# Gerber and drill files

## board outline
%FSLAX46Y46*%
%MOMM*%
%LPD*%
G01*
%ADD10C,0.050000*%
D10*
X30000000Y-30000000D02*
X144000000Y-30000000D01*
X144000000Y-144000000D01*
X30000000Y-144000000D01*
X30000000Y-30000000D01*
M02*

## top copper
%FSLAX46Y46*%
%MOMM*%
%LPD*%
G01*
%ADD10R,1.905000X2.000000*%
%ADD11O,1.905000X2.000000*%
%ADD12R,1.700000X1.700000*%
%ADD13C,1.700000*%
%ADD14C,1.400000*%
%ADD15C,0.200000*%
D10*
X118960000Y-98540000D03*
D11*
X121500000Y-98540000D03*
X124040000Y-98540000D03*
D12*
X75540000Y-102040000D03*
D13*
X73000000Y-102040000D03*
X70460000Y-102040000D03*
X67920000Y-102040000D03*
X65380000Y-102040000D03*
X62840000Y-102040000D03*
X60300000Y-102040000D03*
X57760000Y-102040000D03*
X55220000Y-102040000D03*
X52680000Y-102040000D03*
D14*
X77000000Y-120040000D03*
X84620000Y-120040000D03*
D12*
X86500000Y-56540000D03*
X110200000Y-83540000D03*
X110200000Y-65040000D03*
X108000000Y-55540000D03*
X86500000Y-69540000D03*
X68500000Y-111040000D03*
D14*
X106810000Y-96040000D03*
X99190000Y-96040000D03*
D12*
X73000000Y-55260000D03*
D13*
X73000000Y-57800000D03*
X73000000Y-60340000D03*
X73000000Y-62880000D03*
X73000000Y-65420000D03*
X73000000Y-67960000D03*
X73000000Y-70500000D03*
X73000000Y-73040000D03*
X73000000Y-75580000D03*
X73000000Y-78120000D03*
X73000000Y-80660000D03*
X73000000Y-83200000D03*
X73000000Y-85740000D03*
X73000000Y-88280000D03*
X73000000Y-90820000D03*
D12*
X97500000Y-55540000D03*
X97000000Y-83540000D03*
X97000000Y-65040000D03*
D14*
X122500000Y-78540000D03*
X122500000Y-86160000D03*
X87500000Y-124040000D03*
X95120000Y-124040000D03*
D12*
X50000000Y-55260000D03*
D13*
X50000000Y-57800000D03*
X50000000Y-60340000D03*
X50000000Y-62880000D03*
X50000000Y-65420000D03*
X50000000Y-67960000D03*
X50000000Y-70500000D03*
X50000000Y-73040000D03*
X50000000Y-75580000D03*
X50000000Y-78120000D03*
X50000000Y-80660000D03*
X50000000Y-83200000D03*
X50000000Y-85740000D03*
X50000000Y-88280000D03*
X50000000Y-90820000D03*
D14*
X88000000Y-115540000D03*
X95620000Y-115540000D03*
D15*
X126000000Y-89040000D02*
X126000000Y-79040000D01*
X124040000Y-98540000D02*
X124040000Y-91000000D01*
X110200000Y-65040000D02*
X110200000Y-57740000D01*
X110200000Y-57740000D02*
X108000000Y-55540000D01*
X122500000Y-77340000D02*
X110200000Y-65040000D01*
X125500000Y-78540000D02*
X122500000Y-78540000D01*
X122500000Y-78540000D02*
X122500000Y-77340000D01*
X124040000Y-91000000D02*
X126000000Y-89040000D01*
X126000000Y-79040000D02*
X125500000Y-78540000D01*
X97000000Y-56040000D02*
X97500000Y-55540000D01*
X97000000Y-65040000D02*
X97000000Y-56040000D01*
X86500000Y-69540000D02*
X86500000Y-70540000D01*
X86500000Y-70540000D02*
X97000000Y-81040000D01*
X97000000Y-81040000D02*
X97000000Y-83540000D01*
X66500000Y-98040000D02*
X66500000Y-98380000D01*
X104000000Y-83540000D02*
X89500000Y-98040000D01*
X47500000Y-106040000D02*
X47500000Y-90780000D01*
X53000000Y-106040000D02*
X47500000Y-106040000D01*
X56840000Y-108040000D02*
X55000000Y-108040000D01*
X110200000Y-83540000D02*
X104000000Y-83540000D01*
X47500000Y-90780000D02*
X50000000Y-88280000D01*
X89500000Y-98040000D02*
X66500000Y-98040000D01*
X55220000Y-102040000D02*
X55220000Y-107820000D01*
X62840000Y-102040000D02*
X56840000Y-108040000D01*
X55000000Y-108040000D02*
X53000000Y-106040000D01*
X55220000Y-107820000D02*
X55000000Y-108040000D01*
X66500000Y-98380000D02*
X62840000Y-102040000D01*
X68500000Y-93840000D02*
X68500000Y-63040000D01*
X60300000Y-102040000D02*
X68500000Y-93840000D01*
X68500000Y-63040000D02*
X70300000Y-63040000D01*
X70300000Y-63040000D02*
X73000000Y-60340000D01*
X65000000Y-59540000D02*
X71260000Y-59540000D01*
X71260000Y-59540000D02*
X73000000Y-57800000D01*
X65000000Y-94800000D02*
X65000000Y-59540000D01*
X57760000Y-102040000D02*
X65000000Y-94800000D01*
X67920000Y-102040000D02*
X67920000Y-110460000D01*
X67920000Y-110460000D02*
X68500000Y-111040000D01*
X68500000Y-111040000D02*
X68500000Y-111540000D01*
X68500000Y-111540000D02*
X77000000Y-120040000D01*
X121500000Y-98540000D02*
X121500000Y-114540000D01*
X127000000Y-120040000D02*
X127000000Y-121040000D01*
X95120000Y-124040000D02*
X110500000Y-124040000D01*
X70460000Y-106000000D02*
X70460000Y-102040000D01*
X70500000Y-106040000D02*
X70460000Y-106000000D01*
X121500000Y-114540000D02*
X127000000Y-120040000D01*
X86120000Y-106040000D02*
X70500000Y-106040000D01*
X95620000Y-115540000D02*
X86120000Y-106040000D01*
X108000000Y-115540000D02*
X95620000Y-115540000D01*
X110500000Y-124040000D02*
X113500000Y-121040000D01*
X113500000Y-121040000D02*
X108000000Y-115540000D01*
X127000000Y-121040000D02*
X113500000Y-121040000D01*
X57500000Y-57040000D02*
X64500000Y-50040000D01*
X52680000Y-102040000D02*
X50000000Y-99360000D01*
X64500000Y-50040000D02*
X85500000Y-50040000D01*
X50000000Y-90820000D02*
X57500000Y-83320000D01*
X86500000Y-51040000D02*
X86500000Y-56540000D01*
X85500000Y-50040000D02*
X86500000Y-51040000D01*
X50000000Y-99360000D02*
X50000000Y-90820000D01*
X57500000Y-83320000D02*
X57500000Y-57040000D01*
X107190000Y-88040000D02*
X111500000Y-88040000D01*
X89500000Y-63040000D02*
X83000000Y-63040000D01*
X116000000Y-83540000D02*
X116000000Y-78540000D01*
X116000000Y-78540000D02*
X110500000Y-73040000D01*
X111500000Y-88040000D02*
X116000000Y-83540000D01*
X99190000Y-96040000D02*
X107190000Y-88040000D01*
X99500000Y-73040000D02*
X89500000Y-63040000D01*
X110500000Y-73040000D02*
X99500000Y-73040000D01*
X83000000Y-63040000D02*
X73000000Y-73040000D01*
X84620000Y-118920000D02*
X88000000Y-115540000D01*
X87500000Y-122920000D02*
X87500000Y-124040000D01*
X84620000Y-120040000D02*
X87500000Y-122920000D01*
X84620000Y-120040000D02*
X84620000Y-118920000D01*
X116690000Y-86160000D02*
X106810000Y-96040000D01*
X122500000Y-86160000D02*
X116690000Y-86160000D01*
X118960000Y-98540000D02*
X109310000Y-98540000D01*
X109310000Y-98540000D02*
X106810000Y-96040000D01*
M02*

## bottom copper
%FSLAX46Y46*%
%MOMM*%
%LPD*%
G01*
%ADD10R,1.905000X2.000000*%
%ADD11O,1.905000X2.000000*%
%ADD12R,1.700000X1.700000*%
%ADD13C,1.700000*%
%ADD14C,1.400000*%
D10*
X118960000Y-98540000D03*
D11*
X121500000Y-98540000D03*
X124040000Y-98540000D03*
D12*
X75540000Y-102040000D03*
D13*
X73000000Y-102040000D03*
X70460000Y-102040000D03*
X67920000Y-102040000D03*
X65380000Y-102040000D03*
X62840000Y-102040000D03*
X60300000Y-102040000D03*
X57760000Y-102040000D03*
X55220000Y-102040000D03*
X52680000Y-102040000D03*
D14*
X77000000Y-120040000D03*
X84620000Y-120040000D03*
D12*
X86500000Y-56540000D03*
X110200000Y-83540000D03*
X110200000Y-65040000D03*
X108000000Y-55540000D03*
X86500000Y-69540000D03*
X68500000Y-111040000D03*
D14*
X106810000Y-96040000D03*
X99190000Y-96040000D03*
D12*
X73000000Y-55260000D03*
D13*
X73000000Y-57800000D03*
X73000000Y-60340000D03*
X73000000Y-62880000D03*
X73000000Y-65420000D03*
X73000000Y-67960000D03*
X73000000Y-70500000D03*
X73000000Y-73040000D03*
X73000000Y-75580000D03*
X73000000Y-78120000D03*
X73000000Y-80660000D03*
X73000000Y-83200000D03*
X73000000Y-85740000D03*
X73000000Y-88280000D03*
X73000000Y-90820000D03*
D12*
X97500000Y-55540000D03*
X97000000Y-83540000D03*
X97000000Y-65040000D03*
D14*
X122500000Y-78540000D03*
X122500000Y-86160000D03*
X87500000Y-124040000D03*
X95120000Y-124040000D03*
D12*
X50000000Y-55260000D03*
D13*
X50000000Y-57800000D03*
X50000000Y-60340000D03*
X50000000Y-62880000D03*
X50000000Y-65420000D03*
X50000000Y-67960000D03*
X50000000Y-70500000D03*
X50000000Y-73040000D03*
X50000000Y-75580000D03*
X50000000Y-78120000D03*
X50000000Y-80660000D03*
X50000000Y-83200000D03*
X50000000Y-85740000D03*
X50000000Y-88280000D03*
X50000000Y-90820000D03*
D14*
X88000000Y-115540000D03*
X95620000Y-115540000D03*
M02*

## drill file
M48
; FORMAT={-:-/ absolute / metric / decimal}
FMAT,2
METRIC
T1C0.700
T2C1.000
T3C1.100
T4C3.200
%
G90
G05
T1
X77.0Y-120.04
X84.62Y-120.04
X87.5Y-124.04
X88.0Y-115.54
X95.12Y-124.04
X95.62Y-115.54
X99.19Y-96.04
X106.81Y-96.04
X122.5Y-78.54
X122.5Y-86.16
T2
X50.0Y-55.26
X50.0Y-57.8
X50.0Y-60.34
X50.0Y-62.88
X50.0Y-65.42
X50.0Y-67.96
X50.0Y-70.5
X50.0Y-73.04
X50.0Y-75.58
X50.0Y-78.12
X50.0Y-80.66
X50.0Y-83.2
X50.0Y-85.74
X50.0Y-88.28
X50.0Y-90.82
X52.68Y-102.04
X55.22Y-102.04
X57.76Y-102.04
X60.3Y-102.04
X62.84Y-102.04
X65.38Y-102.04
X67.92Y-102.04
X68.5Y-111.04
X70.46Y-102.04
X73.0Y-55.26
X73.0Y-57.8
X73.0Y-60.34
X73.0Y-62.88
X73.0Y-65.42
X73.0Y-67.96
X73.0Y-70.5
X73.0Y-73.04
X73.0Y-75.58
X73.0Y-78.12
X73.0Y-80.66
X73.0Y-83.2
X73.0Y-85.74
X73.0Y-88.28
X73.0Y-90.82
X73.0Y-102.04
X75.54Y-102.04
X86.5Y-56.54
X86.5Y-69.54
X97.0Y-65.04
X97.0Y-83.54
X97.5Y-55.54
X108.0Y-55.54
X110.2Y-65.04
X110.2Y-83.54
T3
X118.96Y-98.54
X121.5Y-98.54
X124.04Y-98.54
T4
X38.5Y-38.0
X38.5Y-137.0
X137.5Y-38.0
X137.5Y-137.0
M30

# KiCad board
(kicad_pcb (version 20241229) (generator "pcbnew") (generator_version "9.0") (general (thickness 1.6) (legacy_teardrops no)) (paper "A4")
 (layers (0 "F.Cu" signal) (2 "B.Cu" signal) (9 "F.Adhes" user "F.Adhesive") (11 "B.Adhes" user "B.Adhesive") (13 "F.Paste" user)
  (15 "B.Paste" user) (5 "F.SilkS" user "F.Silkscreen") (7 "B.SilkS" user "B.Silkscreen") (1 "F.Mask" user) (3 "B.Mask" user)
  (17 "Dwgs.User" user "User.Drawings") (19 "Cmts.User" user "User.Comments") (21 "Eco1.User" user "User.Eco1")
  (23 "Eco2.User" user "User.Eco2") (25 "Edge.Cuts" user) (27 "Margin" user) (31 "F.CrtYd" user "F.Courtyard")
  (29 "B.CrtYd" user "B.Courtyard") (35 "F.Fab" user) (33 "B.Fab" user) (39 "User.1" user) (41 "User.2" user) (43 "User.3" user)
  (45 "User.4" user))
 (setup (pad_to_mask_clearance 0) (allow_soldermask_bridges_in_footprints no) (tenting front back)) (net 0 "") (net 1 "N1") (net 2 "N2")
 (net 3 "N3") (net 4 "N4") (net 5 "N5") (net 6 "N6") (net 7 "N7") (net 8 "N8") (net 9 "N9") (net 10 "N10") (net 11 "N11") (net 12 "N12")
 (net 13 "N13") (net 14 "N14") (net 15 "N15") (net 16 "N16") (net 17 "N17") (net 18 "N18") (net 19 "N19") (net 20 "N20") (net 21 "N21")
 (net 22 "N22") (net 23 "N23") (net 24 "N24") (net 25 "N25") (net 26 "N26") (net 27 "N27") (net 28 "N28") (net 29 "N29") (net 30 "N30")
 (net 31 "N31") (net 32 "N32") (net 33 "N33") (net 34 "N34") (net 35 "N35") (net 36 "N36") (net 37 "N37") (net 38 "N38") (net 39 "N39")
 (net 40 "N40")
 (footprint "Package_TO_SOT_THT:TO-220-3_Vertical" (layer "F.Cu") (at 118.96 98.54)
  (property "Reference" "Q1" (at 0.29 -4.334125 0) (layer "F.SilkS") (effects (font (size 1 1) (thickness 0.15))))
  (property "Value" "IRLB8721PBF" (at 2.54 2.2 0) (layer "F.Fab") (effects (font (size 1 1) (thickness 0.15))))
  (pad "1" thru_hole rect (at 0 0) (size 1.905 2) (drill 1.1) (layers "*.Cu" "*.Mask") (remove_unused_layers no) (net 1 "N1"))
  (pad "2" thru_hole oval (at 2.54 0) (size 1.905 2) (drill 1.1) (layers "*.Cu" "*.Mask") (remove_unused_layers no) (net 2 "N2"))
  (pad "3" thru_hole oval (at 5.08 0) (size 1.905 2) (drill 1.1) (layers "*.Cu" "*.Mask") (remove_unused_layers no) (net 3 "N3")))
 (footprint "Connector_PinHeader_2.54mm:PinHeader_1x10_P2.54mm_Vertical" (layer "F.Cu") (at 75.54 102.04 -90)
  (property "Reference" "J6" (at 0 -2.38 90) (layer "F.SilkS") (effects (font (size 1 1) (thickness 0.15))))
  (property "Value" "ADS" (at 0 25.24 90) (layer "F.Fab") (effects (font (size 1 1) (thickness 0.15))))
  (pad "1" thru_hole rect (at 0 0 270) (size 1.7 1.7) (drill 1) (layers "*.Cu" "*.Mask") (remove_unused_layers no) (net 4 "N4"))
  (pad "2" thru_hole circle (at 0 2.54 270) (size 1.7 1.7) (drill 1) (layers "*.Cu" "*.Mask") (remove_unused_layers no) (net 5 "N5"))
  (pad "3" thru_hole circle (at 0 5.08 270) (size 1.7 1.7) (drill 1) (layers "*.Cu" "*.Mask") (remove_unused_layers no) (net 2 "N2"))
  (pad "4" thru_hole circle (at 0 7.62 270) (size 1.7 1.7) (drill 1) (layers "*.Cu" "*.Mask") (remove_unused_layers no) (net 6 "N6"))
  (pad "5" thru_hole circle (at 0 10.16 270) (size 1.7 1.7) (drill 1) (layers "*.Cu" "*.Mask") (remove_unused_layers no) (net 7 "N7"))
  (pad "6" thru_hole circle (at 0 12.7 270) (size 1.7 1.7) (drill 1) (layers "*.Cu" "*.Mask") (remove_unused_layers no) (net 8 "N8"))
  (pad "7" thru_hole circle (at 0 15.24 270) (size 1.7 1.7) (drill 1) (layers "*.Cu" "*.Mask") (remove_unused_layers no) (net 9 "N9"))
  (pad "8" thru_hole circle (at 0 17.78 270) (size 1.7 1.7) (drill 1) (layers "*.Cu" "*.Mask") (remove_unused_layers no) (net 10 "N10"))
  (pad "9" thru_hole circle (at 0 20.32 270) (size 1.7 1.7) (drill 1) (layers "*.Cu" "*.Mask") (remove_unused_layers no) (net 8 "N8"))
  (pad "10" thru_hole circle (at 0 22.86 270) (size 1.7 1.7) (drill 1) (layers "*.Cu" "*.Mask") (remove_unused_layers no) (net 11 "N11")))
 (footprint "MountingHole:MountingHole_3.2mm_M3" (layer "F.Cu") (at 137.5 137)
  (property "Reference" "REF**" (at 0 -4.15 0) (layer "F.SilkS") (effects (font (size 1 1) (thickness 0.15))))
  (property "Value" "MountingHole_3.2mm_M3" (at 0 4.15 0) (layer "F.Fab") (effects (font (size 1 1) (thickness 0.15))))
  (pad "" np_thru_hole circle (at 0 0) (size 3.2 3.2) (drill 3.2) (layers "*.Cu" "*.Mask")))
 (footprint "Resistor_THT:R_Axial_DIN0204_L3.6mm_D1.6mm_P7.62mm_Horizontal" (layer "F.Cu") (at 77 120.04)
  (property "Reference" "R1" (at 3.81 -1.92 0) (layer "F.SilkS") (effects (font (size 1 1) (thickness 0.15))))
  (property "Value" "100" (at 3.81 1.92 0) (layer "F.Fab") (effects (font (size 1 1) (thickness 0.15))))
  (pad "1" thru_hole circle (at 0 0) (size 1.4 1.4) (drill 0.7) (layers "*.Cu" "*.Mask") (remove_unused_layers no) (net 6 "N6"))
  (pad "2" thru_hole circle (at 7.62 0) (size 1.4 1.4) (drill 0.7) (layers "*.Cu" "*.Mask") (remove_unused_layers no) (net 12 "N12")))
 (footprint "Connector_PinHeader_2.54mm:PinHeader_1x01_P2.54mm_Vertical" (layer "F.Cu") (at 86.5 56.54 -90)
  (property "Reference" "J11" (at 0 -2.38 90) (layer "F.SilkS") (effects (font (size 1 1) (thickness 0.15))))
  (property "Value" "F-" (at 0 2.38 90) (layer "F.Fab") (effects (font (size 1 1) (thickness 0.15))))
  (pad "1" thru_hole rect (at 0 0 270) (size 1.7 1.7) (drill 1) (layers "*.Cu" "*.Mask") (remove_unused_layers no) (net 11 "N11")))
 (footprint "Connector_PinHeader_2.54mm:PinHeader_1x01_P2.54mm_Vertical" (layer "F.Cu") (at 110.2 83.54)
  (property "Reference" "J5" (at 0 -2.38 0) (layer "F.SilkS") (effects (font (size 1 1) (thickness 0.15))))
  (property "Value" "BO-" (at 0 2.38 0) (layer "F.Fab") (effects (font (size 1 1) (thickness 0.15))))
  (pad "1" thru_hole rect (at 0 0) (size 1.7 1.7) (drill 1) (layers "*.Cu" "*.Mask") (remove_unused_layers no) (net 8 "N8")))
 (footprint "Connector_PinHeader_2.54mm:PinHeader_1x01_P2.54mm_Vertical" (layer "F.Cu") (at 110.2 65.04)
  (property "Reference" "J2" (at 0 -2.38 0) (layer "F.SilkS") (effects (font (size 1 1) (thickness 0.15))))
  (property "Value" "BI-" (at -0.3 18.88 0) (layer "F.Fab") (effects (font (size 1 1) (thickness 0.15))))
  (pad "1" thru_hole rect (at 0 0) (size 1.7 1.7) (drill 1) (layers "*.Cu" "*.Mask") (remove_unused_layers no) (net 3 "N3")))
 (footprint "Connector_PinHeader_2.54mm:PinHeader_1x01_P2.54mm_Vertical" (layer "F.Cu") (at 108 55.54)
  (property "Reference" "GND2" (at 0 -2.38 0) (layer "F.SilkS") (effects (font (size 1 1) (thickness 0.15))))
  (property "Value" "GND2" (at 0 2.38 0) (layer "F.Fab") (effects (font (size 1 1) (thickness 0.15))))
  (pad "1" thru_hole rect (at 0 0) (size 1.7 1.7) (drill 1) (layers "*.Cu" "*.Mask") (remove_unused_layers no) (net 3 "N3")))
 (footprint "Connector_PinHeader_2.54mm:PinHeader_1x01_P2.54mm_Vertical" (layer "F.Cu") (at 86.5 69.54 -90)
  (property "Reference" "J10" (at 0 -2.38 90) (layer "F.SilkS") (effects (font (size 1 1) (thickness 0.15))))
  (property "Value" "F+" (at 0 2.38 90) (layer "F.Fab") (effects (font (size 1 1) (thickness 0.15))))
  (pad "1" thru_hole rect (at 0 0 270) (size 1.7 1.7) (drill 1) (layers "*.Cu" "*.Mask") (remove_unused_layers no) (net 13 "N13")))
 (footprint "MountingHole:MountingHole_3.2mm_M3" (layer "F.Cu") (at 137.5 38)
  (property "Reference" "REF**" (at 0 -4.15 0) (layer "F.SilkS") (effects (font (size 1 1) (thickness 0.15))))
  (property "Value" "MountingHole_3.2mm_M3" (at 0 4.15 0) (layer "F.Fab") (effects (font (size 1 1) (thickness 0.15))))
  (pad "" np_thru_hole circle (at 0 0) (size 3.2 3.2) (drill 3.2) (layers "*.Cu" "*.Mask")))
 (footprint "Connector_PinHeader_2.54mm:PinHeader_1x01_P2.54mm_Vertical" (layer "F.Cu") (at 68.5 111.04)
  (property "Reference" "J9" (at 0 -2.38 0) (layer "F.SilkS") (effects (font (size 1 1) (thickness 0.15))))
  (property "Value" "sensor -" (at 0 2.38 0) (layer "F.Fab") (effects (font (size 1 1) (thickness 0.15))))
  (pad "1" thru_hole rect (at 0 0) (size 1.7 1.7) (drill 1) (layers "*.Cu" "*.Mask") (remove_unused_layers no) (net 6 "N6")))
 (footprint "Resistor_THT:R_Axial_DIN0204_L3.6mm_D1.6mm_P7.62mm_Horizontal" (layer "F.Cu") (at 106.81 96.04 180)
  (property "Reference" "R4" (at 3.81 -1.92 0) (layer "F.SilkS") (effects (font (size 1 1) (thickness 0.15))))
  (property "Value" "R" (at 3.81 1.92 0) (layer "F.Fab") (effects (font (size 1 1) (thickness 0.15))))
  (pad "1" thru_hole circle (at 0 0 180) (size 1.4 1.4) (drill 0.7) (layers "*.Cu" "*.Mask") (remove_unused_layers no) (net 1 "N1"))
  (pad "2" thru_hole circle (at 7.62 0 180) (size 1.4 1.4) (drill 0.7) (layers "*.Cu" "*.Mask") (remove_unused_layers no) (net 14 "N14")))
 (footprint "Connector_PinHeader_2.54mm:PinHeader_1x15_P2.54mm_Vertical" (layer "F.Cu") (at 73 55.26)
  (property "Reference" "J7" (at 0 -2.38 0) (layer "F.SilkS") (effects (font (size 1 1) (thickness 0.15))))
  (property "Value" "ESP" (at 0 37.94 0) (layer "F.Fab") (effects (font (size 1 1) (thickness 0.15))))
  (pad "1" thru_hole rect (at 0 0) (size 1.7 1.7) (drill 1) (layers "*.Cu" "*.Mask") (remove_unused_layers no) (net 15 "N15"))
  (pad "2" thru_hole circle (at 0 2.54) (size 1.7 1.7) (drill 1) (layers "*.Cu" "*.Mask") (remove_unused_layers no) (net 10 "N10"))
  (pad "3" thru_hole circle (at 0 5.08) (size 1.7 1.7) (drill 1) (layers "*.Cu" "*.Mask") (remove_unused_layers no) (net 9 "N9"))
  (pad "4" thru_hole circle (at 0 7.62) (size 1.7 1.7) (drill 1) (layers "*.Cu" "*.Mask") (remove_unused_layers no) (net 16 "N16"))
  (pad "5" thru_hole circle (at 0 10.16) (size 1.7 1.7) (drill 1) (layers "*.Cu" "*.Mask") (remove_unused_layers no) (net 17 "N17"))
  (pad "6" thru_hole circle (at 0 12.7) (size 1.7 1.7) (drill 1) (layers "*.Cu" "*.Mask") (remove_unused_layers no) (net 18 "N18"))
  (pad "7" thru_hole circle (at 0 15.24) (size 1.7 1.7) (drill 1) (layers "*.Cu" "*.Mask") (remove_unused_layers no) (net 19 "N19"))
  (pad "8" thru_hole circle (at 0 17.78) (size 1.7 1.7) (drill 1) (layers "*.Cu" "*.Mask") (remove_unused_layers no) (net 14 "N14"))
  (pad "9" thru_hole circle (at 0 20.32) (size 1.7 1.7) (drill 1) (layers "*.Cu" "*.Mask") (remove_unused_layers no) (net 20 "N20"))
  (pad "10" thru_hole circle (at 0 22.86) (size 1.7 1.7) (drill 1) (layers "*.Cu" "*.Mask") (remove_unused_layers no) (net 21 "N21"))
  (pad "11" thru_hole circle (at 0 25.4) (size 1.7 1.7) (drill 1) (layers "*.Cu" "*.Mask") (remove_unused_layers no) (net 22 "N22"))
  (pad "12" thru_hole circle (at 0 27.94) (size 1.7 1.7) (drill 1) (layers "*.Cu" "*.Mask") (remove_unused_layers no) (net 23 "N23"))
  (pad "13" thru_hole circle (at 0 30.48) (size 1.7 1.7) (drill 1) (layers "*.Cu" "*.Mask") (remove_unused_layers no) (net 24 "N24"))
  (pad "14" thru_hole circle (at 0 33.02) (size 1.7 1.7) (drill 1) (layers "*.Cu" "*.Mask") (remove_unused_layers no) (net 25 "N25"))
  (pad "15" thru_hole circle (at 0 35.56) (size 1.7 1.7) (drill 1) (layers "*.Cu" "*.Mask") (remove_unused_layers no) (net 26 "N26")))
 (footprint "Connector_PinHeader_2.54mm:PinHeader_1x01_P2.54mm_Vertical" (layer "F.Cu") (at 97.5 55.54)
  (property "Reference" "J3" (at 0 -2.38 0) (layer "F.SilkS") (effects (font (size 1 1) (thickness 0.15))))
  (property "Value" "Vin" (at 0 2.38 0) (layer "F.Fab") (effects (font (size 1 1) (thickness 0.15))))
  (pad "1" thru_hole rect (at 0 0) (size 1.7 1.7) (drill 1) (layers "*.Cu" "*.Mask") (remove_unused_layers no) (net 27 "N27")))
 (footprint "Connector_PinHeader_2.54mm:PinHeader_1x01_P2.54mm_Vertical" (layer "F.Cu") (at 97 83.54)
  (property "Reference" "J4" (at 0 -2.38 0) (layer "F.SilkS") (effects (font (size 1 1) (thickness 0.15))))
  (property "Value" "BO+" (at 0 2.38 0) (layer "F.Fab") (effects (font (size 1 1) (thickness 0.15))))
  (pad "1" thru_hole rect (at 0 0) (size 1.7 1.7) (drill 1) (layers "*.Cu" "*.Mask") (remove_unused_layers no) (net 13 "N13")))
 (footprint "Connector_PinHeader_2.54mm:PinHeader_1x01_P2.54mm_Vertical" (layer "F.Cu") (at 97 65.04)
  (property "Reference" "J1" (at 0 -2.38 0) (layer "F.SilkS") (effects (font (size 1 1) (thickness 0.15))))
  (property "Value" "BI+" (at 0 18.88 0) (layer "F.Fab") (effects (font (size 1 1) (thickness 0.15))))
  (pad "1" thru_hole rect (at 0 0) (size 1.7 1.7) (drill 1) (layers "*.Cu" "*.Mask") (remove_unused_layers no) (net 27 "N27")))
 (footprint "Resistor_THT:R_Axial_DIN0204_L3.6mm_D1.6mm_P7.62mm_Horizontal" (layer "F.Cu") (at 122.5 78.54 -90)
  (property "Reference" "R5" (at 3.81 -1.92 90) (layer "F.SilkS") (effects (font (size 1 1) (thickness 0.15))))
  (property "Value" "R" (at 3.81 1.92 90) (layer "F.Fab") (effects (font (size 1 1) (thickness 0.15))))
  (pad "1" thru_hole circle (at 0 0 270) (size 1.4 1.4) (drill 0.7) (layers "*.Cu" "*.Mask") (remove_unused_layers no) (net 3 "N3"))
  (pad "2" thru_hole circle (at 7.62 0 270) (size 1.4 1.4) (drill 0.7) (layers "*.Cu" "*.Mask") (remove_unused_layers no) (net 1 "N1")))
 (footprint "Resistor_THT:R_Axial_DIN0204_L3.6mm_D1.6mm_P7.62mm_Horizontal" (layer "F.Cu") (at 87.5 124.04)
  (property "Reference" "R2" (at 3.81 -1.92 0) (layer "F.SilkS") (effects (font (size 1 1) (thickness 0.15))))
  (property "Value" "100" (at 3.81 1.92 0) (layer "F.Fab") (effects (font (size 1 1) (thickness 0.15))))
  (pad "1" thru_hole circle (at 0 0) (size 1.4 1.4) (drill 0.7) (layers "*.Cu" "*.Mask") (remove_unused_layers no) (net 12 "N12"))
  (pad "2" thru_hole circle (at 7.62 0) (size 1.4 1.4) (drill 0.7) (layers "*.Cu" "*.Mask") (remove_unused_layers no) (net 2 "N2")))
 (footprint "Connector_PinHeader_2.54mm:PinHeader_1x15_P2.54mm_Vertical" (layer "F.Cu") (at 50 55.26)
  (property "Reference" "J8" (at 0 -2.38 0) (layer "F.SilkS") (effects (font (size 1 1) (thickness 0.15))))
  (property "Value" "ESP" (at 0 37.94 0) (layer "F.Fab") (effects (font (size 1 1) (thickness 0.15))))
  (pad "1" thru_hole rect (at 0 0) (size 1.7 1.7) (drill 1) (layers "*.Cu" "*.Mask") (remove_unused_layers no) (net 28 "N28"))
  (pad "2" thru_hole circle (at 0 2.54) (size 1.7 1.7) (drill 1) (layers "*.Cu" "*.Mask") (remove_unused_layers no) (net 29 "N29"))
  (pad "3" thru_hole circle (at 0 5.08) (size 1.7 1.7) (drill 1) (layers "*.Cu" "*.Mask") (remove_unused_layers no) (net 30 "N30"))
  (pad "4" thru_hole circle (at 0 7.62) (size 1.7 1.7) (drill 1) (layers "*.Cu" "*.Mask") (remove_unused_layers no) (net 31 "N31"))
  (pad "5" thru_hole circle (at 0 10.16) (size 1.7 1.7) (drill 1) (layers "*.Cu" "*.Mask") (remove_unused_layers no) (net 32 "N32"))
  (pad "6" thru_hole circle (at 0 12.7) (size 1.7 1.7) (drill 1) (layers "*.Cu" "*.Mask") (remove_unused_layers no) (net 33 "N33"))
  (pad "7" thru_hole circle (at 0 15.24) (size 1.7 1.7) (drill 1) (layers "*.Cu" "*.Mask") (remove_unused_layers no) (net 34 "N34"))
  (pad "8" thru_hole circle (at 0 17.78) (size 1.7 1.7) (drill 1) (layers "*.Cu" "*.Mask") (remove_unused_layers no) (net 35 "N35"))
  (pad "9" thru_hole circle (at 0 20.32) (size 1.7 1.7) (drill 1) (layers "*.Cu" "*.Mask") (remove_unused_layers no) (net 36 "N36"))
  (pad "10" thru_hole circle (at 0 22.86) (size 1.7 1.7) (drill 1) (layers "*.Cu" "*.Mask") (remove_unused_layers no) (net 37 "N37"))
  (pad "11" thru_hole circle (at 0 25.4) (size 1.7 1.7) (drill 1) (layers "*.Cu" "*.Mask") (remove_unused_layers no) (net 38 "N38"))
  (pad "12" thru_hole circle (at 0 27.94) (size 1.7 1.7) (drill 1) (layers "*.Cu" "*.Mask") (remove_unused_layers no) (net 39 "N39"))
  (pad "13" thru_hole circle (at 0 30.48) (size 1.7 1.7) (drill 1) (layers "*.Cu" "*.Mask") (remove_unused_layers no) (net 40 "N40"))
  (pad "14" thru_hole circle (at 0 33.02) (size 1.7 1.7) (drill 1) (layers "*.Cu" "*.Mask") (remove_unused_layers no) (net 8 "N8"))
  (pad "15" thru_hole circle (at 0 35.56) (size 1.7 1.7) (drill 1) (layers "*.Cu" "*.Mask") (remove_unused_layers no) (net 11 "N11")))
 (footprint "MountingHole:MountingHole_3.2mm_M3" (layer "F.Cu") (at 38.5 137)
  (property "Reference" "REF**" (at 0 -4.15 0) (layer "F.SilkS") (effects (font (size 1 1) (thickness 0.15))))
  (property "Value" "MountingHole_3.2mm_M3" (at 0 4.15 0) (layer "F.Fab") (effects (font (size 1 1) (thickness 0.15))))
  (pad "" np_thru_hole circle (at 0 0) (size 3.2 3.2) (drill 3.2) (layers "*.Cu" "*.Mask")))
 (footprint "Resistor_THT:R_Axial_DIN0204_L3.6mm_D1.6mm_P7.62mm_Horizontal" (layer "F.Cu") (at 88 115.54)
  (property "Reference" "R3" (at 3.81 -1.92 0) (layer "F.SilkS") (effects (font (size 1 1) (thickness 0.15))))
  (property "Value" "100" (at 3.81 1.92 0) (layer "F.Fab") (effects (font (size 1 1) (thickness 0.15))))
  (pad "1" thru_hole circle (at 0 0) (size 1.4 1.4) (drill 0.7) (layers "*.Cu" "*.Mask") (remove_unused_layers no) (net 12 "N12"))
  (pad "2" thru_hole circle (at 7.62 0) (size 1.4 1.4) (drill 0.7) (layers "*.Cu" "*.Mask") (remove_unused_layers no) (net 2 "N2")))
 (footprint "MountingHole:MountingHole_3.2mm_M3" (layer "F.Cu") (at 38.5 38)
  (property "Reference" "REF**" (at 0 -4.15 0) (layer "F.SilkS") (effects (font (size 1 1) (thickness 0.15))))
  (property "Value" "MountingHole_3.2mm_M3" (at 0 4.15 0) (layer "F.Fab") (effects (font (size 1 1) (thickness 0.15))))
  (pad "" np_thru_hole circle (at 0 0) (size 3.2 3.2) (drill 3.2) (layers "*.Cu" "*.Mask")))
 (gr_rect (start 30 30) (end 144 144) (stroke (width 0.05) (type solid)) (fill no) (layer "Edge.Cuts"))
 (segment (start 126 89.04) (end 126 79.04) (width 0.2) (layer "F.Cu") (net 3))
 (segment (start 124.04 98.54) (end 124.04 91) (width 0.2) (layer "F.Cu") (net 3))
 (segment (start 110.2 65.04) (end 110.2 57.74) (width 0.2) (layer "F.Cu") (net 3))
 (segment (start 110.2 57.74) (end 108 55.54) (width 0.2) (layer "F.Cu") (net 3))
 (segment (start 122.5 77.34) (end 110.2 65.04) (width 0.2) (layer "F.Cu") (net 3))
 (segment (start 125.5 78.54) (end 122.5 78.54) (width 0.2) (layer "F.Cu") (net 3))
 (segment (start 122.5 78.54) (end 122.5 77.34) (width 0.2) (layer "F.Cu") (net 3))
 (segment (start 124.04 91) (end 126 89.04) (width 0.2) (layer "F.Cu") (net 3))
 (segment (start 126 79.04) (end 125.5 78.54) (width 0.2) (layer "F.Cu") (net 3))
 (segment (start 97 56.04) (end 97.5 55.54) (width 0.2) (layer "F.Cu") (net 27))
 (segment (start 97 65.04) (end 97 56.04) (width 0.2) (layer "F.Cu") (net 27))
 (segment (start 86.5 69.54) (end 86.5 70.54) (width 0.2) (layer "F.Cu") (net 13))
 (segment (start 86.5 70.54) (end 97 81.04) (width 0.2) (layer "F.Cu") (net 13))
 (segment (start 97 81.04) (end 97 83.54) (width 0.2) (layer "F.Cu") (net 13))
 (segment (start 66.5 98.04) (end 66.5 98.38) (width 0.2) (layer "F.Cu") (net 8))
 (segment (start 104 83.54) (end 89.5 98.04) (width 0.2) (layer "F.Cu") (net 8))
 (segment (start 47.5 106.04) (end 47.5 90.78) (width 0.2) (layer "F.Cu") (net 8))
 (segment (start 53 106.04) (end 47.5 106.04) (width 0.2) (layer "F.Cu") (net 8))
 (segment (start 56.84 108.04) (end 55 108.04) (width 0.2) (layer "F.Cu") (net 8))
 (segment (start 110.2 83.54) (end 104 83.54) (width 0.2) (layer "F.Cu") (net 8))
 (segment (start 47.5 90.78) (end 50 88.28) (width 0.2) (layer "F.Cu") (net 8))
 (segment (start 89.5 98.04) (end 66.5 98.04) (width 0.2) (layer "F.Cu") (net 8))
 (segment (start 55.22 102.04) (end 55.22 107.82) (width 0.2) (layer "F.Cu") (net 8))
 (segment (start 62.84 102.04) (end 56.84 108.04) (width 0.2) (layer "F.Cu") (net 8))
 (segment (start 55 108.04) (end 53 106.04) (width 0.2) (layer "F.Cu") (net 8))
 (segment (start 55.22 107.82) (end 55 108.04) (width 0.2) (layer "F.Cu") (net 8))
 (segment (start 66.5 98.38) (end 62.84 102.04) (width 0.2) (layer "F.Cu") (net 8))
 (segment (start 68.5 93.84) (end 68.5 63.04) (width 0.2) (layer "F.Cu") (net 9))
 (segment (start 60.3 102.04) (end 68.5 93.84) (width 0.2) (layer "F.Cu") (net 9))
 (segment (start 68.5 63.04) (end 70.3 63.04) (width 0.2) (layer "F.Cu") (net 9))
 (segment (start 70.3 63.04) (end 73 60.34) (width 0.2) (layer "F.Cu") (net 9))
 (segment (start 65 59.54) (end 71.26 59.54) (width 0.2) (layer "F.Cu") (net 10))
 (segment (start 71.26 59.54) (end 73 57.8) (width 0.2) (layer "F.Cu") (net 10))
 (segment (start 65 94.8) (end 65 59.54) (width 0.2) (layer "F.Cu") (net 10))
 (segment (start 57.76 102.04) (end 65 94.8) (width 0.2) (layer "F.Cu") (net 10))
 (segment (start 67.92 102.04) (end 67.92 110.46) (width 0.2) (layer "F.Cu") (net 6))
 (segment (start 67.92 110.46) (end 68.5 111.04) (width 0.2) (layer "F.Cu") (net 6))
 (segment (start 68.5 111.04) (end 68.5 111.54) (width 0.2) (layer "F.Cu") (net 6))
 (segment (start 68.5 111.54) (end 77 120.04) (width 0.2) (layer "F.Cu") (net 6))
 (segment (start 121.5 98.54) (end 121.5 114.54) (width 0.2) (layer "F.Cu") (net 2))
 (segment (start 127 120.04) (end 127 121.04) (width 0.2) (layer "F.Cu") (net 2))
 (segment (start 95.12 124.04) (end 110.5 124.04) (width 0.2) (layer "F.Cu") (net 2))
 (segment (start 70.46 106) (end 70.46 102.04) (width 0.2) (layer "F.Cu") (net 2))
 (segment (start 70.5 106.04) (end 70.46 106) (width 0.2) (layer "F.Cu") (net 2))
 (segment (start 121.5 114.54) (end 127 120.04) (width 0.2) (layer "F.Cu") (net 2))
 (segment (start 86.12 106.04) (end 70.5 106.04) (width 0.2) (layer "F.Cu") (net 2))
 (segment (start 95.62 115.54) (end 86.12 106.04) (width 0.2) (layer "F.Cu") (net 2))
 (segment (start 108 115.54) (end 95.62 115.54) (width 0.2) (layer "F.Cu") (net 2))
 (segment (start 110.5 124.04) (end 113.5 121.04) (width 0.2) (layer "F.Cu") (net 2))
 (segment (start 113.5 121.04) (end 108 115.54) (width 0.2) (layer "F.Cu") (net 2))
 (segment (start 127 121.04) (end 113.5 121.04) (width 0.2) (layer "F.Cu") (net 2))
 (segment (start 57.5 57.04) (end 64.5 50.04) (width 0.2) (layer "F.Cu") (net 11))
 (segment (start 52.68 102.04) (end 50 99.36) (width 0.2) (layer "F.Cu") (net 11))
 (segment (start 64.5 50.04) (end 85.5 50.04) (width 0.2) (layer "F.Cu") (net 11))
 (segment (start 50 90.82) (end 57.5 83.32) (width 0.2) (layer "F.Cu") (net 11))
 (segment (start 86.5 51.04) (end 86.5 56.54) (width 0.2) (layer "F.Cu") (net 11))
 (segment (start 85.5 50.04) (end 86.5 51.04) (width 0.2) (layer "F.Cu") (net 11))
 (segment (start 50 99.36) (end 50 90.82) (width 0.2) (layer "F.Cu") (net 11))
 (segment (start 57.5 83.32) (end 57.5 57.04) (width 0.2) (layer "F.Cu") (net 11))
 (segment (start 107.19 88.04) (end 111.5 88.04) (width 0.2) (layer "F.Cu") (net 14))
 (segment (start 89.5 63.04) (end 83 63.04) (width 0.2) (layer "F.Cu") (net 14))
 (segment (start 116 83.54) (end 116 78.54) (width 0.2) (layer "F.Cu") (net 14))
 (segment (start 116 78.54) (end 110.5 73.04) (width 0.2) (layer "F.Cu") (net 14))
 (segment (start 111.5 88.04) (end 116 83.54) (width 0.2) (layer "F.Cu") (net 14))
 (segment (start 99.19 96.04) (end 107.19 88.04) (width 0.2) (layer "F.Cu") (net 14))
 (segment (start 99.5 73.04) (end 89.5 63.04) (width 0.2) (layer "F.Cu") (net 14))
 (segment (start 110.5 73.04) (end 99.5 73.04) (width 0.2) (layer "F.Cu") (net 14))
 (segment (start 83 63.04) (end 73 73.04) (width 0.2) (layer "F.Cu") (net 14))
 (segment (start 84.62 118.92) (end 88 115.54) (width 0.2) (layer "F.Cu") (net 12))
 (segment (start 87.5 122.92) (end 87.5 124.04) (width 0.2) (layer "F.Cu") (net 12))
 (segment (start 84.62 120.04) (end 87.5 122.92) (width 0.2) (layer "F.Cu") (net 12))
 (segment (start 84.62 120.04) (end 84.62 118.92) (width 0.2) (layer "F.Cu") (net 12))
 (segment (start 116.69 86.16) (end 106.81 96.04) (width 0.2) (layer "F.Cu") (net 1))
 (segment (start 122.5 86.16) (end 116.69 86.16) (width 0.2) (layer "F.Cu") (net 1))
 (segment (start 118.96 98.54) (end 109.31 98.54) (width 0.2) (layer "F.Cu") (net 1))
 (segment (start 109.31 98.54) (end 106.81 96.04) (width 0.2) (layer "F.Cu") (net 1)))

